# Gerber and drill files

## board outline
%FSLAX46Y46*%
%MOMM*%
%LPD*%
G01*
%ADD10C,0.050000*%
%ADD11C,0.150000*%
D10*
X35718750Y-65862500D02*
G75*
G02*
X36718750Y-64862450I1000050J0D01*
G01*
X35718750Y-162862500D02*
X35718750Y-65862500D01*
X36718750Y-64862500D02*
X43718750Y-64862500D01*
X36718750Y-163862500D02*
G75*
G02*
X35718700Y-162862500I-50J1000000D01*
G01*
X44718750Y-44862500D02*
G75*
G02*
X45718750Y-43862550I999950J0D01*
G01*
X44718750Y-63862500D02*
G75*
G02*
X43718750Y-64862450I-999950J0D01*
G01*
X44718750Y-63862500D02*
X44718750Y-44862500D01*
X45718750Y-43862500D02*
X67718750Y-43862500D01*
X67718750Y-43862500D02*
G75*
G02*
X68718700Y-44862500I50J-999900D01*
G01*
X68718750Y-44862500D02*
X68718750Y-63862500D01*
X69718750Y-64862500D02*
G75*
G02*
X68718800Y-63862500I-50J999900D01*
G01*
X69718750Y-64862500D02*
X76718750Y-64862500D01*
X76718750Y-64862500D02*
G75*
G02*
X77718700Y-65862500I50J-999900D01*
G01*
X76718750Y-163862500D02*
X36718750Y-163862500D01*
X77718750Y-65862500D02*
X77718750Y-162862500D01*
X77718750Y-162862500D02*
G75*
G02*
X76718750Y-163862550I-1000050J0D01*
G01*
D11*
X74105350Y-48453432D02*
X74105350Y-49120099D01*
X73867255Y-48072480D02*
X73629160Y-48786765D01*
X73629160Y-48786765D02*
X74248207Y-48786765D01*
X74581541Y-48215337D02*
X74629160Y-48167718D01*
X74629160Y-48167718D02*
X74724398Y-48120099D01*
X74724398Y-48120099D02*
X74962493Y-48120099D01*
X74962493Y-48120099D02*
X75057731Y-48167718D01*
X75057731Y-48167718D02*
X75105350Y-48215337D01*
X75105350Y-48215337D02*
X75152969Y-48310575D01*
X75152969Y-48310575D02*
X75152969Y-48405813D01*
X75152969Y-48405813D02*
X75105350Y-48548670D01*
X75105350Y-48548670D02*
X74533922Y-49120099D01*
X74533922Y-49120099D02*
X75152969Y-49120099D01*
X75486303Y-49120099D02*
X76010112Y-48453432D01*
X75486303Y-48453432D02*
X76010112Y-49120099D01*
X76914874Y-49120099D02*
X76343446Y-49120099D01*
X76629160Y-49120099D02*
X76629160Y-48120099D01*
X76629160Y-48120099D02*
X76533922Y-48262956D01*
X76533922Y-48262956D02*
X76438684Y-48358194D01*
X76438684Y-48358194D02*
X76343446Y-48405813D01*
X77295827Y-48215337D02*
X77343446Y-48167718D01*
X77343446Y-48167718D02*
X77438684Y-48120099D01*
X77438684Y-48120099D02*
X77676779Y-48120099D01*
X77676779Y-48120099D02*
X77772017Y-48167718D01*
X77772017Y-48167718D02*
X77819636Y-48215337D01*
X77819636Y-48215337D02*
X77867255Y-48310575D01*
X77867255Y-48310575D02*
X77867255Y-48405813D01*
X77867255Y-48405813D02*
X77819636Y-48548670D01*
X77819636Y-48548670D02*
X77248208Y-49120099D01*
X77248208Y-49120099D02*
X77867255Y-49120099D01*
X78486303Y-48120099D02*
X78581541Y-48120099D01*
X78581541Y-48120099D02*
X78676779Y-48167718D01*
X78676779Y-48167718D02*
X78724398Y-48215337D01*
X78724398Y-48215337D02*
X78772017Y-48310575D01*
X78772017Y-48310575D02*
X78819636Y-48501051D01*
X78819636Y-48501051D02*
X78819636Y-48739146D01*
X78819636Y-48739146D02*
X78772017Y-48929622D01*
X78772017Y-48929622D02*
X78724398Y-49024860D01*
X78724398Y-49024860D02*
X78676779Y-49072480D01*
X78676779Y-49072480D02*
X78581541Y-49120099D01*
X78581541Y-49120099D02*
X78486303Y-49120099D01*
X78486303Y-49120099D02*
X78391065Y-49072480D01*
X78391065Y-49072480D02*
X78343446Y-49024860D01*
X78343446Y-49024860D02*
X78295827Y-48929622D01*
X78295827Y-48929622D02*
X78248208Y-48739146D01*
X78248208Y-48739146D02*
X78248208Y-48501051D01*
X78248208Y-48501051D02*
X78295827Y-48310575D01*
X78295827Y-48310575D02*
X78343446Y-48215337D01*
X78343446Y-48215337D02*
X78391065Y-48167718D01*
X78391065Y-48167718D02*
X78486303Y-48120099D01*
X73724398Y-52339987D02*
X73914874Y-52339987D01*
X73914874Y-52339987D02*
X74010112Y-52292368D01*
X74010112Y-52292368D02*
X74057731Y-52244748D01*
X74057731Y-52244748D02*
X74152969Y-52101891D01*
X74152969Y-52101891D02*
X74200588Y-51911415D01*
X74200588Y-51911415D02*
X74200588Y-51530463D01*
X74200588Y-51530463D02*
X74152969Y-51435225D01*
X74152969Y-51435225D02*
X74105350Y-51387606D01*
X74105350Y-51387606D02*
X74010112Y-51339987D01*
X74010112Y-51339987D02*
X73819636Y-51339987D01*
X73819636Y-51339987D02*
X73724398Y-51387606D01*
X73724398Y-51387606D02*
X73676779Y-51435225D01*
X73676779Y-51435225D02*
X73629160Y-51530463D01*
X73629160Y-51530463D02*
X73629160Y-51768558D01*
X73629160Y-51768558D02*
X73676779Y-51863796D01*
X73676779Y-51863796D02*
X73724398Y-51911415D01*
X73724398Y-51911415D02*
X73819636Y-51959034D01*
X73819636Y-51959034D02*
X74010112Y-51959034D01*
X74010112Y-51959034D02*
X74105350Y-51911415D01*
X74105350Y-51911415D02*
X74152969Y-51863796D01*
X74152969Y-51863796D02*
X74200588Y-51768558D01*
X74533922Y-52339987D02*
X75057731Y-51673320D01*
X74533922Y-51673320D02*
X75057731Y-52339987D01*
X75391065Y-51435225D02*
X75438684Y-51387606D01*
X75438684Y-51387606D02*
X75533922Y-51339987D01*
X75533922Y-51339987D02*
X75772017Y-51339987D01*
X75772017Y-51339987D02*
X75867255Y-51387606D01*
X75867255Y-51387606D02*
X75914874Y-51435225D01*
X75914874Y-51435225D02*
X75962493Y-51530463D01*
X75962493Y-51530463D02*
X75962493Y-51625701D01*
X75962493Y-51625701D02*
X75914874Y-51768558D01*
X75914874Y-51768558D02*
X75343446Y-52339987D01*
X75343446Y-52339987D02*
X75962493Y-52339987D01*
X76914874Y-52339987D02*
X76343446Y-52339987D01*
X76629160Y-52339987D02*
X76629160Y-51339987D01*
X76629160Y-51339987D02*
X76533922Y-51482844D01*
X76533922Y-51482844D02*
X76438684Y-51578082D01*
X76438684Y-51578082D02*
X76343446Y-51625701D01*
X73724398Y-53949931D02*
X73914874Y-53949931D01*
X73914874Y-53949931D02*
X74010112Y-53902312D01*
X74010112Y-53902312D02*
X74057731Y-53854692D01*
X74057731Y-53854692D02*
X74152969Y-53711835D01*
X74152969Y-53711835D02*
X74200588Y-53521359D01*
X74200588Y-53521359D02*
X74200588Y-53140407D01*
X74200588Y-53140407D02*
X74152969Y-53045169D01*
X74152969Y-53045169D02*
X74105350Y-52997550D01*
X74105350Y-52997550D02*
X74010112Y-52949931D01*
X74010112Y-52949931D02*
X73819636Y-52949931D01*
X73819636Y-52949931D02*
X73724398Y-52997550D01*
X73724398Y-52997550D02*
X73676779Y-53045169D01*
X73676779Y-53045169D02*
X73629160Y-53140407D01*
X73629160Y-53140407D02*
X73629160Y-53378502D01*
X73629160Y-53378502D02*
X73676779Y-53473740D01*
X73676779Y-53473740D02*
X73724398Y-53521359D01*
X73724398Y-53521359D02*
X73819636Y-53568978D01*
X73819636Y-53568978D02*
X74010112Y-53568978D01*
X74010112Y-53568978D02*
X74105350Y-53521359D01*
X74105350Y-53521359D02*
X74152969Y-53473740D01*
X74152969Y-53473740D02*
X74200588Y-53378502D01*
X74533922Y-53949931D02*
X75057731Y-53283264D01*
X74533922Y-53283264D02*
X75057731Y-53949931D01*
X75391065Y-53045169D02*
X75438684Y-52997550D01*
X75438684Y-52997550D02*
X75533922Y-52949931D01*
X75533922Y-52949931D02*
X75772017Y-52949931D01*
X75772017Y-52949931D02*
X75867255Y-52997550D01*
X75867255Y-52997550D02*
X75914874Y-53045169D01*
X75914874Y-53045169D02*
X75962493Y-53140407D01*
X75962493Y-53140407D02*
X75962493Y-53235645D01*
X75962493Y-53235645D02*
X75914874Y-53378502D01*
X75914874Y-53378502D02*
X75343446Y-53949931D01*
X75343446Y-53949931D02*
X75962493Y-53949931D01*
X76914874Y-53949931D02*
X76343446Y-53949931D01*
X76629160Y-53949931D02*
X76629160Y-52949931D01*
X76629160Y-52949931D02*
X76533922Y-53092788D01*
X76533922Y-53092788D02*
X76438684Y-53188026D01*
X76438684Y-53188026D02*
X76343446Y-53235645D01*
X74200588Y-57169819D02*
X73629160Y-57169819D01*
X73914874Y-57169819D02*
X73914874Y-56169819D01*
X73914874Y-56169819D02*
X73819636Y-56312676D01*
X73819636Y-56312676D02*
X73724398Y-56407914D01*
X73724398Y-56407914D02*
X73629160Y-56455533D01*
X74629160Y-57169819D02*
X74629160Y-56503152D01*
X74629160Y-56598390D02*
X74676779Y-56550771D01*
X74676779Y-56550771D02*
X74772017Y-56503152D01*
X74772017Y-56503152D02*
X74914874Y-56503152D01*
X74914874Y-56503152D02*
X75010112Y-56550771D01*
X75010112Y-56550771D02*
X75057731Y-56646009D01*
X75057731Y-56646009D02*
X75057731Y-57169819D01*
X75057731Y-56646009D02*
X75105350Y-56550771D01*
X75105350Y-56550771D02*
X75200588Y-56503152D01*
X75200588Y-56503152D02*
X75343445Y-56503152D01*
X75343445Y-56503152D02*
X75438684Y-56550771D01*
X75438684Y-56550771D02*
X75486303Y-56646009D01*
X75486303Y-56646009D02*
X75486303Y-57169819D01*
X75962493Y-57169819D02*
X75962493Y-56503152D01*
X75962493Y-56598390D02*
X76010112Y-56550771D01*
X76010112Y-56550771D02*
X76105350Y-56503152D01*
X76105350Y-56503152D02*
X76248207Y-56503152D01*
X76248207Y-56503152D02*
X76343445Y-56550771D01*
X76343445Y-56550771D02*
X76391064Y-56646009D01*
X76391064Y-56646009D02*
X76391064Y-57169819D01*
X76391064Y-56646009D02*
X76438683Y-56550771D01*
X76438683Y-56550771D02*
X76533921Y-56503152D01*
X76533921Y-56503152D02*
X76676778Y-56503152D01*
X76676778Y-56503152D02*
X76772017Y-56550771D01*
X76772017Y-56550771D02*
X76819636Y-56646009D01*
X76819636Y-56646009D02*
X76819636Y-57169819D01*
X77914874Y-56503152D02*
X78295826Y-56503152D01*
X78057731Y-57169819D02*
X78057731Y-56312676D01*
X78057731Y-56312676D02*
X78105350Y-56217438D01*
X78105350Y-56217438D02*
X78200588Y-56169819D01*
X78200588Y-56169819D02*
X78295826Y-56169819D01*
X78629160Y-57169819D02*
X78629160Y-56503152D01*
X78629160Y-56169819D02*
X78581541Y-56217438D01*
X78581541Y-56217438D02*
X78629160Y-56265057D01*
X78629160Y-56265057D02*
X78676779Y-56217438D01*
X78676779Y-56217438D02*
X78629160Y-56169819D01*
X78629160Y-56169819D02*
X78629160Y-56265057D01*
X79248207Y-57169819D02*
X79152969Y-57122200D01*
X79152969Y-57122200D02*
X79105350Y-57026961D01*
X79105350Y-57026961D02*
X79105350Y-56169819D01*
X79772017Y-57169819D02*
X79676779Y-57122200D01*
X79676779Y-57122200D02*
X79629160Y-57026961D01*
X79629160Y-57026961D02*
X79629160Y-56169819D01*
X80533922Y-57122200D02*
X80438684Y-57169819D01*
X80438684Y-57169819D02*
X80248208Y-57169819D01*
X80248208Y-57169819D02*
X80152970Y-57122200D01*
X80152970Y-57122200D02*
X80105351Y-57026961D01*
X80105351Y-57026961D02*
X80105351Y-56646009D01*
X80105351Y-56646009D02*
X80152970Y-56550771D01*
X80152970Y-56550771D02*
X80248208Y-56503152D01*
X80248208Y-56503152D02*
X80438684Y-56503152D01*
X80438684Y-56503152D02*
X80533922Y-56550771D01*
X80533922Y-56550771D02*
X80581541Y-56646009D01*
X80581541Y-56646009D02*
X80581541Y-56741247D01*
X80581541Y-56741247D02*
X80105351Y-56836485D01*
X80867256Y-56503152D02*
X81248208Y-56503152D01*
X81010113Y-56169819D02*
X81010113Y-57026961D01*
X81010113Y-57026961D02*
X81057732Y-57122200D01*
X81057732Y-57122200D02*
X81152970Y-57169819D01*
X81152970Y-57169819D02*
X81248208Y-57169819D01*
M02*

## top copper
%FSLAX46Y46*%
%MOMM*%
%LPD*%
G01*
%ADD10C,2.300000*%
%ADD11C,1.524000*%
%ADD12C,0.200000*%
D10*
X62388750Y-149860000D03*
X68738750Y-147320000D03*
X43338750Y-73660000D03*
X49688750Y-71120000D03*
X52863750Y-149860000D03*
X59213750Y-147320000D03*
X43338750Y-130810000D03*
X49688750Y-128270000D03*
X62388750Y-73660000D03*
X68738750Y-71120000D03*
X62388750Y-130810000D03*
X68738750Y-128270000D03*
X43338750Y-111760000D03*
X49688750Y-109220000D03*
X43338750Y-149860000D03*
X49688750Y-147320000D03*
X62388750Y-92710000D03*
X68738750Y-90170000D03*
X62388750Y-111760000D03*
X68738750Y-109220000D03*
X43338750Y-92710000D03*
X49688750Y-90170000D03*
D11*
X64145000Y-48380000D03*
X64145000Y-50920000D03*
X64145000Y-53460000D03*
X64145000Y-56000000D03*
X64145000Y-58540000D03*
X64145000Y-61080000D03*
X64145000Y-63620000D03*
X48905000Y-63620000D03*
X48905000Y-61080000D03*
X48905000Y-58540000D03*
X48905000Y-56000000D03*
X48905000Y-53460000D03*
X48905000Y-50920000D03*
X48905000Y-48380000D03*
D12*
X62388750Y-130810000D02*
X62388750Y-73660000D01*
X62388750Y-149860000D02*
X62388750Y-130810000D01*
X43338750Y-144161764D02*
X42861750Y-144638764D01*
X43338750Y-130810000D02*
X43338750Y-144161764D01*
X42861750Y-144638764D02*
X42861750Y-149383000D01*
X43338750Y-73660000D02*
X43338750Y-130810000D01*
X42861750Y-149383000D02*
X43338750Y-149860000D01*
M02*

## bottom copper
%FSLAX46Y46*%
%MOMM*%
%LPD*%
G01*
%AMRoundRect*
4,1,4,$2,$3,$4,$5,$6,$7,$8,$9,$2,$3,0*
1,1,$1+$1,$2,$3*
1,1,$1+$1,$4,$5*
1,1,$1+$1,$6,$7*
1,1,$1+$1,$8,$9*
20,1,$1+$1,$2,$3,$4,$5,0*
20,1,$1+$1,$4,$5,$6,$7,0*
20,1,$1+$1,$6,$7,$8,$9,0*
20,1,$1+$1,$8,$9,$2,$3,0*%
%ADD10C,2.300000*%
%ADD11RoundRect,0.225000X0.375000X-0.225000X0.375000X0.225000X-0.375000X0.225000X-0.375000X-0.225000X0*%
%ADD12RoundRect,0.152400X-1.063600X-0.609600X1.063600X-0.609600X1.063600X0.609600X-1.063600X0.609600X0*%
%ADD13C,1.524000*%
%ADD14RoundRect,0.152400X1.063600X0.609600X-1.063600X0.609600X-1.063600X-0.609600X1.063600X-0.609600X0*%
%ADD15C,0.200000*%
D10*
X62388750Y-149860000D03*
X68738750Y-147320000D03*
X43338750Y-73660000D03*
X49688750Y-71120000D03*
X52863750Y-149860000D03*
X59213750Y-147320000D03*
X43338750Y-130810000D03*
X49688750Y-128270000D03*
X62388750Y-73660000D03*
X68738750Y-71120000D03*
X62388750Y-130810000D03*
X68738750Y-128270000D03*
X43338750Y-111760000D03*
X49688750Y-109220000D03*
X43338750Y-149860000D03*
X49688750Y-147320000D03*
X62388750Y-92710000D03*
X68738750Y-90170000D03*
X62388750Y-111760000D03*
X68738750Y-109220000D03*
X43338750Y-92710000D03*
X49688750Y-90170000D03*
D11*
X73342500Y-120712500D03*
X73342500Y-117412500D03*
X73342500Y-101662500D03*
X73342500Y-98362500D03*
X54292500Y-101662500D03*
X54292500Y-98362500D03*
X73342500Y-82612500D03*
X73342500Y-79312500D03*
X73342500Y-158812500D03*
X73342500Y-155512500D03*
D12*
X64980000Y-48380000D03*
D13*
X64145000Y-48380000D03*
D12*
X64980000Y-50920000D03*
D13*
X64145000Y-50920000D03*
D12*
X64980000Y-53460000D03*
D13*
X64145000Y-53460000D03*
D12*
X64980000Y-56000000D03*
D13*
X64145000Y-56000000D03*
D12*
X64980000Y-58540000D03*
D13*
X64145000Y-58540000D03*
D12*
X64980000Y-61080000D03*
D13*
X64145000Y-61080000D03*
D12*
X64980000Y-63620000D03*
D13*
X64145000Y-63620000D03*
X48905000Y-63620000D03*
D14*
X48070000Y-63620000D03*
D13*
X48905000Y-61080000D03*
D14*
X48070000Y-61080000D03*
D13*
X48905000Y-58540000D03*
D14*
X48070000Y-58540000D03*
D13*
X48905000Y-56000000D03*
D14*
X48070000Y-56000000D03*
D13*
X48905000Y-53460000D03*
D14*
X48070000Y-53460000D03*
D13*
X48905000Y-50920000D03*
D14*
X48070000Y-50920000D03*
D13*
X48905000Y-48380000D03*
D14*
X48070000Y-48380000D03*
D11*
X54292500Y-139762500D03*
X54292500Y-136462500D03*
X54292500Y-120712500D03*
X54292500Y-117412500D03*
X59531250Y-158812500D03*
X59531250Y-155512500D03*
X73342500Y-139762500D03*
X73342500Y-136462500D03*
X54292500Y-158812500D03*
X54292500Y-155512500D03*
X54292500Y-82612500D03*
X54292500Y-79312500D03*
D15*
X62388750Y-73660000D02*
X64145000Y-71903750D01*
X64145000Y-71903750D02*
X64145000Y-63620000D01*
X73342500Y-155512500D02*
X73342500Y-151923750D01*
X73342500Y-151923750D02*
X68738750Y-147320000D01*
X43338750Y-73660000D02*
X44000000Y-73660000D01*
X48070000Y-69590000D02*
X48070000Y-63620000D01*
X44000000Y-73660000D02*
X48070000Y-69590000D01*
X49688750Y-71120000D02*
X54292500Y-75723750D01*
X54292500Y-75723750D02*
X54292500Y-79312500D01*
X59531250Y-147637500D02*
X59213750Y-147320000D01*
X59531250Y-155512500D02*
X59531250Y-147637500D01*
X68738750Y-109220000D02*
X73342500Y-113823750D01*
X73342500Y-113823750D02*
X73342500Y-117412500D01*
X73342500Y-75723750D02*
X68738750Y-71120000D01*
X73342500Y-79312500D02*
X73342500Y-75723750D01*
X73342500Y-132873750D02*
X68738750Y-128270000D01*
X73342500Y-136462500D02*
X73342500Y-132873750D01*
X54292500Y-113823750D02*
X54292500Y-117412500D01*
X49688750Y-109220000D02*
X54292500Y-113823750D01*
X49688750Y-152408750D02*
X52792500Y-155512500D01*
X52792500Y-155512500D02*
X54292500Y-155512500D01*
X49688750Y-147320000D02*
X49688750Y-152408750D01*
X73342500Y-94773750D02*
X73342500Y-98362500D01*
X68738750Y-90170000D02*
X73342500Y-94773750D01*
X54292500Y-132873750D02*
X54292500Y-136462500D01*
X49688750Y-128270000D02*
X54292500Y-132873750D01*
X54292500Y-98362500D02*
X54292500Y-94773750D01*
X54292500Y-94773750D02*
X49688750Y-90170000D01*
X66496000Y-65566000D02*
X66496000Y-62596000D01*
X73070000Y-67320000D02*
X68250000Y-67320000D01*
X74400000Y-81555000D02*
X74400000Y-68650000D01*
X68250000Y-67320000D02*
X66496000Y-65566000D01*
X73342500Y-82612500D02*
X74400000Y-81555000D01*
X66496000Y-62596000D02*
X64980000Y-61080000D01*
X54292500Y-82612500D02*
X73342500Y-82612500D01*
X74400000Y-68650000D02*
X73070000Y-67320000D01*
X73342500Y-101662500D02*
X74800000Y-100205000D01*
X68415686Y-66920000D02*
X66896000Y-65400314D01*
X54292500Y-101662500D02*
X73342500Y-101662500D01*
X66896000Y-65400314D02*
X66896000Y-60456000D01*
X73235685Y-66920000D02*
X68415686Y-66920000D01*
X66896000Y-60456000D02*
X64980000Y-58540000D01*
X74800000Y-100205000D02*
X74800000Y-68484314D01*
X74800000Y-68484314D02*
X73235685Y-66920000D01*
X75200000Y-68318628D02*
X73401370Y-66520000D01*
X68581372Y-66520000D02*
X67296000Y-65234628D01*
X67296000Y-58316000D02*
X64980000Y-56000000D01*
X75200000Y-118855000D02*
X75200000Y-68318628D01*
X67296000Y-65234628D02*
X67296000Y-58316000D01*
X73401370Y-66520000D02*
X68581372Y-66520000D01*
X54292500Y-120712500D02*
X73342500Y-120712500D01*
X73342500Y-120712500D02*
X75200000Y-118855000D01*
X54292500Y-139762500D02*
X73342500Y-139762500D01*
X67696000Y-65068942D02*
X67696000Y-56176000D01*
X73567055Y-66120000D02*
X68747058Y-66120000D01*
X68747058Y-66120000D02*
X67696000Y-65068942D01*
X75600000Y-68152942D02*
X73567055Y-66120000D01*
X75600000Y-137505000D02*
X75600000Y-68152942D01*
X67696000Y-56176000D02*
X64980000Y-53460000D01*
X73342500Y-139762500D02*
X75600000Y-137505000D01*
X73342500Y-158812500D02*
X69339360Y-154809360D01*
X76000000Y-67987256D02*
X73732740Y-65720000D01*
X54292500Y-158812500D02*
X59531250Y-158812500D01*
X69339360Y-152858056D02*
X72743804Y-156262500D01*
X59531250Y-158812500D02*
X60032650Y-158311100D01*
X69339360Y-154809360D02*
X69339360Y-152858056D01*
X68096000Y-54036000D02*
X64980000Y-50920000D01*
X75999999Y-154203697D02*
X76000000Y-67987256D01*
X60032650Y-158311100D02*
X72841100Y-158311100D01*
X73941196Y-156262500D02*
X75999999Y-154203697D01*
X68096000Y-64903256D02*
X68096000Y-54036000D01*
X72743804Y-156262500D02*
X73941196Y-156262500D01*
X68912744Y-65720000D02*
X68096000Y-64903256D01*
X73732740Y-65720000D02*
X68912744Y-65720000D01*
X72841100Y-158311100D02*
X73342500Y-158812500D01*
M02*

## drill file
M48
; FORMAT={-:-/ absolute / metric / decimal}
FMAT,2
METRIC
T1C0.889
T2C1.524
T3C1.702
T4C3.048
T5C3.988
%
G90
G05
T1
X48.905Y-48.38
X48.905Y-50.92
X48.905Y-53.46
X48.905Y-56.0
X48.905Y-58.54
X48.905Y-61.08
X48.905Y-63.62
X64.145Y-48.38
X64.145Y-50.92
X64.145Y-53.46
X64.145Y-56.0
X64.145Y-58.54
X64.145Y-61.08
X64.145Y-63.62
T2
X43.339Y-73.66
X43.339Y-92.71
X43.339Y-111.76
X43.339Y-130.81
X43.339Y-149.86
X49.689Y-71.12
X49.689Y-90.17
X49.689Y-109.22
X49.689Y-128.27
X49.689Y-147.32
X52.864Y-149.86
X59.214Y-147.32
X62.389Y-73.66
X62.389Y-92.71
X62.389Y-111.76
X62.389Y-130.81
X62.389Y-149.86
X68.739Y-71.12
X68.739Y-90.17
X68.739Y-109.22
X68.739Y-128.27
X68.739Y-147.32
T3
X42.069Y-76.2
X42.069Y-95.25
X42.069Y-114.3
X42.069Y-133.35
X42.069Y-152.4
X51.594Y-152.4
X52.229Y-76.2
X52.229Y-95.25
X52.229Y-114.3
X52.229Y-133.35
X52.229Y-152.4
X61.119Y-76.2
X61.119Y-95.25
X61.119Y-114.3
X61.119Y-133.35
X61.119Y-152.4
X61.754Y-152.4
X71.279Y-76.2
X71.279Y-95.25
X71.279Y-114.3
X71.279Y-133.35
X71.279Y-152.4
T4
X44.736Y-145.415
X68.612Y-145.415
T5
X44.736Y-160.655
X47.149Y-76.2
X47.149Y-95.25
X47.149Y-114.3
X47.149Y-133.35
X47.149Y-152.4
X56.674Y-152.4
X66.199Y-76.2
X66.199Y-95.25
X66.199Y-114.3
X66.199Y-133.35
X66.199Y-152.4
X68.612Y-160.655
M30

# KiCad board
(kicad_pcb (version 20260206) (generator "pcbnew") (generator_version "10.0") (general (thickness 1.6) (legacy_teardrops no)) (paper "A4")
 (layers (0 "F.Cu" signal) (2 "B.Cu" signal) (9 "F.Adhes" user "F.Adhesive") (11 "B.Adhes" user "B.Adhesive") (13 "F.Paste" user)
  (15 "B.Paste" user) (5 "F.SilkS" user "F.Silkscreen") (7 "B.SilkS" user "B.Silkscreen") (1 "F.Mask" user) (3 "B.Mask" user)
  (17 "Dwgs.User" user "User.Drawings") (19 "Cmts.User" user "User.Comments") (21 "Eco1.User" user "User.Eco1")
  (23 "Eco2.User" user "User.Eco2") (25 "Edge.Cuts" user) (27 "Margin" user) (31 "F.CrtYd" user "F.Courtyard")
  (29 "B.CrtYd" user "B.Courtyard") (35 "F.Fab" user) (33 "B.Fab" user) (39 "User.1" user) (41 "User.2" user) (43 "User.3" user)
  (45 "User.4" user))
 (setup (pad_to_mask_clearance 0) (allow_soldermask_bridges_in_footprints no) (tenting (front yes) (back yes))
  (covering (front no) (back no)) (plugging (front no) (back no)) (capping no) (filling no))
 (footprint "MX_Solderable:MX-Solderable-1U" (layer "F.Cu") (at 66.19875 152.4)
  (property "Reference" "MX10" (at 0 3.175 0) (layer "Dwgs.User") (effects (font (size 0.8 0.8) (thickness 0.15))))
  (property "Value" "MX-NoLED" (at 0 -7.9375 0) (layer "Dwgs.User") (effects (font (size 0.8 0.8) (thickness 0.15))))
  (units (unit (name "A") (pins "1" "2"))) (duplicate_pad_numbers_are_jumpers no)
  (pad "" np_thru_hole circle (at -5.08 0 48.099) (size 1.7018 1.7018) (drill 1.7018) (layers "*.Cu" "*.Mask"))
  (pad "" np_thru_hole circle (at 0 0) (size 3.9878 3.9878) (drill 3.9878) (layers "*.Cu" "*.Mask"))
  (pad "" np_thru_hole circle (at 5.08 0 48.099) (size 1.7018 1.7018) (drill 1.7018) (layers "*.Cu" "*.Mask"))
  (pad "1" thru_hole circle (at -3.81 -2.54) (size 2.3 2.3) (drill 1.524) (layers "*.Cu" "B.Mask") (remove_unused_layers no) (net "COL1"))
  (pad "2" thru_hole circle (at 2.54 -5.08) (size 2.3 2.3) (drill 1.524) (layers "*.Cu" "B.Mask") (remove_unused_layers no)
   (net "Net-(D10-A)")))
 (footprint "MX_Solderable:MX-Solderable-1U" (layer "F.Cu") (at 47.14875 76.2)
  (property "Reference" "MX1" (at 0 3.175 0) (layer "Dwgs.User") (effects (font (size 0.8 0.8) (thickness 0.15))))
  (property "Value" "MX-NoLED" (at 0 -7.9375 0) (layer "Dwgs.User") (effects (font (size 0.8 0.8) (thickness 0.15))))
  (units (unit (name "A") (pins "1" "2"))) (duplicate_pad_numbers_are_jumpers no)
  (pad "" np_thru_hole circle (at -5.08 0 48.099) (size 1.7018 1.7018) (drill 1.7018) (layers "*.Cu" "*.Mask"))
  (pad "" np_thru_hole circle (at 0 0) (size 3.9878 3.9878) (drill 3.9878) (layers "*.Cu" "*.Mask"))
  (pad "" np_thru_hole circle (at 5.08 0 48.099) (size 1.7018 1.7018) (drill 1.7018) (layers "*.Cu" "*.Mask"))
  (pad "1" thru_hole circle (at -3.81 -2.54) (size 2.3 2.3) (drill 1.524) (layers "*.Cu" "B.Mask") (remove_unused_layers no) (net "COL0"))
  (pad "2" thru_hole circle (at 2.54 -5.08) (size 2.3 2.3) (drill 1.524) (layers "*.Cu" "B.Mask") (remove_unused_layers no)
   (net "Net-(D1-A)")))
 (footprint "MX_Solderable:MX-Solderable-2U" (layer "F.Cu") (at 56.67375 152.4)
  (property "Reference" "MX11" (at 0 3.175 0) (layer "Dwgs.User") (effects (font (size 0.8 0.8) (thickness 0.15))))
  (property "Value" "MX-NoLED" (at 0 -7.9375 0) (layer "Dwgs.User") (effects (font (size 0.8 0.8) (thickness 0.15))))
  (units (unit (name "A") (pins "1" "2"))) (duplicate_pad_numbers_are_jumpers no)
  (pad "" np_thru_hole circle (at -11.938 -6.985) (size 3.048 3.048) (drill 3.048) (layers "*.Cu" "*.Mask"))
  (pad "" np_thru_hole circle (at -11.938 8.255) (size 3.9878 3.9878) (drill 3.9878) (layers "*.Cu" "*.Mask"))
  (pad "" np_thru_hole circle (at -5.08 0 48.099) (size 1.7018 1.7018) (drill 1.7018) (layers "*.Cu" "*.Mask"))
  (pad "" np_thru_hole circle (at 0 0) (size 3.9878 3.9878) (drill 3.9878) (layers "*.Cu" "*.Mask"))
  (pad "" np_thru_hole circle (at 5.08 0 48.099) (size 1.7018 1.7018) (drill 1.7018) (layers "*.Cu" "*.Mask"))
  (pad "" np_thru_hole circle (at 11.938 -6.985) (size 3.048 3.048) (drill 3.048) (layers "*.Cu" "*.Mask"))
  (pad "" np_thru_hole circle (at 11.938 8.255) (size 3.9878 3.9878) (drill 3.9878) (layers "*.Cu" "*.Mask"))
  (pad "1" thru_hole circle (at -3.81 -2.54) (size 2.3 2.3) (drill 1.524) (layers "*.Cu" "B.Mask") (remove_unused_layers no)
   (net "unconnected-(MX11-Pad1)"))
  (pad "2" thru_hole circle (at 2.54 -5.08) (size 2.3 2.3) (drill 1.524) (layers "*.Cu" "B.Mask") (remove_unused_layers no)
   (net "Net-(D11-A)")))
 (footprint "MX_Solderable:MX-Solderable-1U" (layer "F.Cu") (at 47.14875 133.35)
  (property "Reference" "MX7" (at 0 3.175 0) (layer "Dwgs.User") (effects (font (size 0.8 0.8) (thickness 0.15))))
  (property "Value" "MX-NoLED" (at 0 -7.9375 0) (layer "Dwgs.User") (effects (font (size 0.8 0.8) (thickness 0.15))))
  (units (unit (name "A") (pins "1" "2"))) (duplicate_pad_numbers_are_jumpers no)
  (pad "" np_thru_hole circle (at -5.08 0 48.099) (size 1.7018 1.7018) (drill 1.7018) (layers "*.Cu" "*.Mask"))
  (pad "" np_thru_hole circle (at 0 0) (size 3.9878 3.9878) (drill 3.9878) (layers "*.Cu" "*.Mask"))
  (pad "" np_thru_hole circle (at 5.08 0 48.099) (size 1.7018 1.7018) (drill 1.7018) (layers "*.Cu" "*.Mask"))
  (pad "1" thru_hole circle (at -3.81 -2.54) (size 2.3 2.3) (drill 1.524) (layers "*.Cu" "B.Mask") (remove_unused_layers no) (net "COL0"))
  (pad "2" thru_hole circle (at 2.54 -5.08) (size 2.3 2.3) (drill 1.524) (layers "*.Cu" "B.Mask") (remove_unused_layers no)
   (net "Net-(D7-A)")))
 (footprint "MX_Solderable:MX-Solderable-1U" (layer "F.Cu") (at 66.19875 76.2)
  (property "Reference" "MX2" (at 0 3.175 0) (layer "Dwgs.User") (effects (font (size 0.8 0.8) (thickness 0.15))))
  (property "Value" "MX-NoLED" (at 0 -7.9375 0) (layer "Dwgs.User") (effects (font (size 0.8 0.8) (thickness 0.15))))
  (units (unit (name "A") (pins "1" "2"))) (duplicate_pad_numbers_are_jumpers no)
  (pad "" np_thru_hole circle (at -5.08 0 48.099) (size 1.7018 1.7018) (drill 1.7018) (layers "*.Cu" "*.Mask"))
  (pad "" np_thru_hole circle (at 0 0) (size 3.9878 3.9878) (drill 3.9878) (layers "*.Cu" "*.Mask"))
  (pad "" np_thru_hole circle (at 5.08 0 48.099) (size 1.7018 1.7018) (drill 1.7018) (layers "*.Cu" "*.Mask"))
  (pad "1" thru_hole circle (at -3.81 -2.54) (size 2.3 2.3) (drill 1.524) (layers "*.Cu" "B.Mask") (remove_unused_layers no) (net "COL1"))
  (pad "2" thru_hole circle (at 2.54 -5.08) (size 2.3 2.3) (drill 1.524) (layers "*.Cu" "B.Mask") (remove_unused_layers no)
   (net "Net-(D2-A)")))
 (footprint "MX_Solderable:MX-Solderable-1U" (layer "F.Cu") (at 66.19875 133.35)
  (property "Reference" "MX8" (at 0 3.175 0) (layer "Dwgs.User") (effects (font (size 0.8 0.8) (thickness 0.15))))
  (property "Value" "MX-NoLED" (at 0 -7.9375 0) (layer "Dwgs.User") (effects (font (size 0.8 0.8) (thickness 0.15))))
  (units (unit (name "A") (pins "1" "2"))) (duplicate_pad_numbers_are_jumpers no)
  (pad "" np_thru_hole circle (at -5.08 0 48.099) (size 1.7018 1.7018) (drill 1.7018) (layers "*.Cu" "*.Mask"))
  (pad "" np_thru_hole circle (at 0 0) (size 3.9878 3.9878) (drill 3.9878) (layers "*.Cu" "*.Mask"))
  (pad "" np_thru_hole circle (at 5.08 0 48.099) (size 1.7018 1.7018) (drill 1.7018) (layers "*.Cu" "*.Mask"))
  (pad "1" thru_hole circle (at -3.81 -2.54) (size 2.3 2.3) (drill 1.524) (layers "*.Cu" "B.Mask") (remove_unused_layers no) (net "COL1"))
  (pad "2" thru_hole circle (at 2.54 -5.08) (size 2.3 2.3) (drill 1.524) (layers "*.Cu" "B.Mask") (remove_unused_layers no)
   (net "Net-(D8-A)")))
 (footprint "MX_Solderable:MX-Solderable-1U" (layer "F.Cu") (at 47.14875 114.3)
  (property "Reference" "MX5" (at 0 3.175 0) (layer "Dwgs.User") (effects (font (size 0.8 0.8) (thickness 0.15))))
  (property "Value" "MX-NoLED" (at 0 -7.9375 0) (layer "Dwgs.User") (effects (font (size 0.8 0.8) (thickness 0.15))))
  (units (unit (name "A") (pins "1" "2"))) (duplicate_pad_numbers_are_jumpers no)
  (pad "" np_thru_hole circle (at -5.08 0 48.099) (size 1.7018 1.7018) (drill 1.7018) (layers "*.Cu" "*.Mask"))
  (pad "" np_thru_hole circle (at 0 0) (size 3.9878 3.9878) (drill 3.9878) (layers "*.Cu" "*.Mask"))
  (pad "" np_thru_hole circle (at 5.08 0 48.099) (size 1.7018 1.7018) (drill 1.7018) (layers "*.Cu" "*.Mask"))
  (pad "1" thru_hole circle (at -3.81 -2.54) (size 2.3 2.3) (drill 1.524) (layers "*.Cu" "B.Mask") (remove_unused_layers no) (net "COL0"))
  (pad "2" thru_hole circle (at 2.54 -5.08) (size 2.3 2.3) (drill 1.524) (layers "*.Cu" "B.Mask") (remove_unused_layers no)
   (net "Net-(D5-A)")))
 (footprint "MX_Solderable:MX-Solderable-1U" (layer "F.Cu") (at 47.14875 152.4)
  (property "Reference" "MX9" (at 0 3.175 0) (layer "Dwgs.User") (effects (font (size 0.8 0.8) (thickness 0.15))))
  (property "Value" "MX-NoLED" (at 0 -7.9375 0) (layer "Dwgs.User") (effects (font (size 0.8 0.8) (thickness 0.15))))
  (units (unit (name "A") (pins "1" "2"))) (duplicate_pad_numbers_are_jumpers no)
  (pad "" np_thru_hole circle (at -5.08 0 48.099) (size 1.7018 1.7018) (drill 1.7018) (layers "*.Cu" "*.Mask"))
  (pad "" np_thru_hole circle (at 0 0) (size 3.9878 3.9878) (drill 3.9878) (layers "*.Cu" "*.Mask"))
  (pad "" np_thru_hole circle (at 5.08 0 48.099) (size 1.7018 1.7018) (drill 1.7018) (layers "*.Cu" "*.Mask"))
  (pad "1" thru_hole circle (at -3.81 -2.54) (size 2.3 2.3) (drill 1.524) (layers "*.Cu" "B.Mask") (remove_unused_layers no) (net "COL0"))
  (pad "2" thru_hole circle (at 2.54 -5.08) (size 2.3 2.3) (drill 1.524) (layers "*.Cu" "B.Mask") (remove_unused_layers no)
   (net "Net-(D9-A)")))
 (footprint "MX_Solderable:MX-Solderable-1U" (layer "F.Cu") (at 66.19875 95.25)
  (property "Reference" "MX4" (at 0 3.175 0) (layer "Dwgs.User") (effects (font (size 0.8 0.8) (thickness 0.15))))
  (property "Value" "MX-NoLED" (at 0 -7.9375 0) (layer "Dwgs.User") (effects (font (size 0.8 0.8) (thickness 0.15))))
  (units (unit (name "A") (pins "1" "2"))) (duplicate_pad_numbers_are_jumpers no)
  (pad "" np_thru_hole circle (at -5.08 0 48.099) (size 1.7018 1.7018) (drill 1.7018) (layers "*.Cu" "*.Mask"))
  (pad "" np_thru_hole circle (at 0 0) (size 3.9878 3.9878) (drill 3.9878) (layers "*.Cu" "*.Mask"))
  (pad "" np_thru_hole circle (at 5.08 0 48.099) (size 1.7018 1.7018) (drill 1.7018) (layers "*.Cu" "*.Mask"))
  (pad "1" thru_hole circle (at -3.81 -2.54) (size 2.3 2.3) (drill 1.524) (layers "*.Cu" "B.Mask") (remove_unused_layers no) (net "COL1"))
  (pad "2" thru_hole circle (at 2.54 -5.08) (size 2.3 2.3) (drill 1.524) (layers "*.Cu" "B.Mask") (remove_unused_layers no)
   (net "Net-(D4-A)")))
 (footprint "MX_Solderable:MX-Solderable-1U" (layer "F.Cu") (at 66.19875 114.3)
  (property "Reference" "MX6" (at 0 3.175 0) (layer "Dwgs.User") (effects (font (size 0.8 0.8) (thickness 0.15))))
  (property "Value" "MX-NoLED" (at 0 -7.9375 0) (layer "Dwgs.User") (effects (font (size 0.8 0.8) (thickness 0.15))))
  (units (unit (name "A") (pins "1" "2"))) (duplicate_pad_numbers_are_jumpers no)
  (pad "" np_thru_hole circle (at -5.08 0 48.099) (size 1.7018 1.7018) (drill 1.7018) (layers "*.Cu" "*.Mask"))
  (pad "" np_thru_hole circle (at 0 0) (size 3.9878 3.9878) (drill 3.9878) (layers "*.Cu" "*.Mask"))
  (pad "" np_thru_hole circle (at 5.08 0 48.099) (size 1.7018 1.7018) (drill 1.7018) (layers "*.Cu" "*.Mask"))
  (pad "1" thru_hole circle (at -3.81 -2.54) (size 2.3 2.3) (drill 1.524) (layers "*.Cu" "B.Mask") (remove_unused_layers no) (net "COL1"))
  (pad "2" thru_hole circle (at 2.54 -5.08) (size 2.3 2.3) (drill 1.524) (layers "*.Cu" "B.Mask") (remove_unused_layers no)
   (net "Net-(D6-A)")))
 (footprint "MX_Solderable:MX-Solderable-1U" (layer "F.Cu") (at 47.14875 95.25)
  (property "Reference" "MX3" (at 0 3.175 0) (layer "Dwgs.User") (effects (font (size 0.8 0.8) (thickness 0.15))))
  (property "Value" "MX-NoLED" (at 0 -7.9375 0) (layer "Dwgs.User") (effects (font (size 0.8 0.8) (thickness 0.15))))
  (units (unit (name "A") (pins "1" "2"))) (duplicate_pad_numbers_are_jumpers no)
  (pad "" np_thru_hole circle (at -5.08 0 48.099) (size 1.7018 1.7018) (drill 1.7018) (layers "*.Cu" "*.Mask"))
  (pad "" np_thru_hole circle (at 0 0) (size 3.9878 3.9878) (drill 3.9878) (layers "*.Cu" "*.Mask"))
  (pad "" np_thru_hole circle (at 5.08 0 48.099) (size 1.7018 1.7018) (drill 1.7018) (layers "*.Cu" "*.Mask"))
  (pad "1" thru_hole circle (at -3.81 -2.54) (size 2.3 2.3) (drill 1.524) (layers "*.Cu" "B.Mask") (remove_unused_layers no) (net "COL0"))
  (pad "2" thru_hole circle (at 2.54 -5.08) (size 2.3 2.3) (drill 1.524) (layers "*.Cu" "B.Mask") (remove_unused_layers no)
   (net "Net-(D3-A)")))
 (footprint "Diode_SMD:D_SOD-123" (layer "B.Cu") (at 73.3425 119.0625 90)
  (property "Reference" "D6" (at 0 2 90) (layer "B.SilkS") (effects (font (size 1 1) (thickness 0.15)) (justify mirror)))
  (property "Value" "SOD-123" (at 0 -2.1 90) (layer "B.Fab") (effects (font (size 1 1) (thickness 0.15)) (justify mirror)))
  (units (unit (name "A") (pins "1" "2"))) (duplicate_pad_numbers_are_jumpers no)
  (pad "1" smd roundrect (at -1.65 0 90) (size 0.9 1.2) (layers "B.Cu" "B.Mask" "B.Paste") (roundrect_rratio 0.25) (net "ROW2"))
  (pad "2" smd roundrect (at 1.65 0 90) (size 0.9 1.2) (layers "B.Cu" "B.Mask" "B.Paste") (roundrect_rratio 0.25) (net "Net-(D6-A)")))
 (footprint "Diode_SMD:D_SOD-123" (layer "B.Cu") (at 73.3425 100.0125 90)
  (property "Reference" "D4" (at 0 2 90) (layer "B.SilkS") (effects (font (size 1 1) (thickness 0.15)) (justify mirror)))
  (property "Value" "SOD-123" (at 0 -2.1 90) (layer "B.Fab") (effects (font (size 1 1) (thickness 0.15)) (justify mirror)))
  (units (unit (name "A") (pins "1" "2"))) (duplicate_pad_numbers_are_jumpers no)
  (pad "1" smd roundrect (at -1.65 0 90) (size 0.9 1.2) (layers "B.Cu" "B.Mask" "B.Paste") (roundrect_rratio 0.25) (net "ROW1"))
  (pad "2" smd roundrect (at 1.65 0 90) (size 0.9 1.2) (layers "B.Cu" "B.Mask" "B.Paste") (roundrect_rratio 0.25) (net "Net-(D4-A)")))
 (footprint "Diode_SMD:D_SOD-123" (layer "B.Cu") (at 54.2925 100.0125 90)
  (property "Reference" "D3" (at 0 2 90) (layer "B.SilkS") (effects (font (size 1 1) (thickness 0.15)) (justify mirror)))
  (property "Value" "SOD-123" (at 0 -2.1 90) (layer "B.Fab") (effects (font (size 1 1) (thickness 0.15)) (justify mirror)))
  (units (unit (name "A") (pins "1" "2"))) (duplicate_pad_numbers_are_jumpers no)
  (pad "1" smd roundrect (at -1.65 0 90) (size 0.9 1.2) (layers "B.Cu" "B.Mask" "B.Paste") (roundrect_rratio 0.25) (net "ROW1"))
  (pad "2" smd roundrect (at 1.65 0 90) (size 0.9 1.2) (layers "B.Cu" "B.Mask" "B.Paste") (roundrect_rratio 0.25) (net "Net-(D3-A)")))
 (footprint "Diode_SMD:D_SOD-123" (layer "B.Cu") (at 73.3425 80.9625 90)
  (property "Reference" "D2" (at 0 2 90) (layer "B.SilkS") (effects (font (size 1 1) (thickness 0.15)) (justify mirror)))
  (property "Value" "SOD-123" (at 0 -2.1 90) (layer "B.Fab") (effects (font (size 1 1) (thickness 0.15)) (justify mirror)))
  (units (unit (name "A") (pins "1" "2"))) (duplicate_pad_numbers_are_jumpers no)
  (pad "1" smd roundrect (at -1.65 0 90) (size 0.9 1.2) (layers "B.Cu" "B.Mask" "B.Paste") (roundrect_rratio 0.25) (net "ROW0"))
  (pad "2" smd roundrect (at 1.65 0 90) (size 0.9 1.2) (layers "B.Cu" "B.Mask" "B.Paste") (roundrect_rratio 0.25) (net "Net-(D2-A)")))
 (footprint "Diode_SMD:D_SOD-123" (layer "B.Cu") (at 73.3425 157.1625 90)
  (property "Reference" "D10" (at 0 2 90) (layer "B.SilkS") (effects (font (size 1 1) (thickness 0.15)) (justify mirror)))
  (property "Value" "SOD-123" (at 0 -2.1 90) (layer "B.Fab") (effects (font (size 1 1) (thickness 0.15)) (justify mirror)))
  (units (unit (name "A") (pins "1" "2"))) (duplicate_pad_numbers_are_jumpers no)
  (pad "1" smd roundrect (at -1.65 0 90) (size 0.9 1.2) (layers "B.Cu" "B.Mask" "B.Paste") (roundrect_rratio 0.25) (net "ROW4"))
  (pad "2" smd roundrect (at 1.65 0 90) (size 0.9 1.2) (layers "B.Cu" "B.Mask" "B.Paste") (roundrect_rratio 0.25) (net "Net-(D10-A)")))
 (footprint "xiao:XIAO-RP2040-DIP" (layer "B.Cu") (at 56.525 56 180)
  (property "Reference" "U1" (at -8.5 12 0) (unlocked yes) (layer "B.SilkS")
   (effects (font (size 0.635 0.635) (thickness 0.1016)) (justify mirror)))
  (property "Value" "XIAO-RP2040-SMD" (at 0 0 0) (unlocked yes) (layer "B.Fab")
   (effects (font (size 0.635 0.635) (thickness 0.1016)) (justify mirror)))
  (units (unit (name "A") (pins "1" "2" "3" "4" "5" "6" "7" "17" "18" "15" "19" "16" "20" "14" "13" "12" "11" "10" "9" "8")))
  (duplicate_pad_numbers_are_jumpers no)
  (pad "1" smd roundrect (at -8.455 7.62) (size 2.432 1.524) (layers "B.Cu" "B.Mask") (roundrect_rratio 0.1)
   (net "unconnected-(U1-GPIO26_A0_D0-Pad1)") (thermal_bridge_angle 45))
  (pad "1" thru_hole circle (at -7.62 7.62) (size 1.524 1.524) (drill 0.889) (layers "*.Cu" "*.Mask") (remove_unused_layers no)
   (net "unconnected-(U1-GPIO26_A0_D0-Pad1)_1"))
  (pad "2" smd roundrect (at -8.455 5.08) (size 2.432 1.524) (layers "B.Cu" "B.Mask") (roundrect_rratio 0.1) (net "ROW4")
   (thermal_bridge_angle 45))
  (pad "2" thru_hole circle (at -7.62 5.08) (size 1.524 1.524) (drill 0.889) (layers "*.Cu" "*.Mask") (remove_unused_layers no) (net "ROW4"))
  (pad "3" smd roundrect (at -8.455 2.54) (size 2.432 1.524) (layers "B.Cu" "B.Mask") (roundrect_rratio 0.1) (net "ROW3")
   (thermal_bridge_angle 45))
  (pad "3" thru_hole circle (at -7.62 2.54) (size 1.524 1.524) (drill 0.889) (layers "*.Cu" "*.Mask") (remove_unused_layers no) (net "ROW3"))
  (pad "4" smd roundrect (at -8.455 0) (size 2.432 1.524) (layers "B.Cu" "B.Mask") (roundrect_rratio 0.1) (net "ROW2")
   (thermal_bridge_angle 45))
  (pad "4" thru_hole circle (at -7.62 0) (size 1.524 1.524) (drill 0.889) (layers "*.Cu" "*.Mask") (remove_unused_layers no) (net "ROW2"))
  (pad "5" smd roundrect (at -8.455 -2.54) (size 2.432 1.524) (layers "B.Cu" "B.Mask") (roundrect_rratio 0.1) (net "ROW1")
   (thermal_bridge_angle 45))
  (pad "5" thru_hole circle (at -7.62 -2.54) (size 1.524 1.524) (drill 0.889) (layers "*.Cu" "*.Mask") (remove_unused_layers no)
   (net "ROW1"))
  (pad "6" smd roundrect (at -8.455 -5.08) (size 2.432 1.524) (layers "B.Cu" "B.Mask") (roundrect_rratio 0.1) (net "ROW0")
   (thermal_bridge_angle 45))
  (pad "6" thru_hole circle (at -7.62 -5.08) (size 1.524 1.524) (drill 0.889) (layers "*.Cu" "*.Mask") (remove_unused_layers no)
   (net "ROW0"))
  (pad "7" smd roundrect (at -8.455 -7.62) (size 2.432 1.524) (layers "B.Cu" "B.Mask") (roundrect_rratio 0.1) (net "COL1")
   (thermal_bridge_angle 45))
  (pad "7" thru_hole circle (at -7.62 -7.62) (size 1.524 1.524) (drill 0.889) (layers "*.Cu" "*.Mask") (remove_unused_layers no)
   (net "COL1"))
  (pad "8" thru_hole circle (at 7.62 -7.62 180) (size 1.524 1.524) (drill 0.889) (layers "*.Cu" "*.Mask") (remove_unused_layers no)
   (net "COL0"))
  (pad "8" smd roundrect (at 8.455 -7.62 180) (size 2.432 1.524) (layers "B.Cu" "B.Mask") (roundrect_rratio 0.1) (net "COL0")
   (thermal_bridge_angle 45))
  (pad "9" thru_hole circle (at 7.62 -5.08 180) (size 1.524 1.524) (drill 0.889) (layers "*.Cu" "*.Mask") (remove_unused_layers no)
   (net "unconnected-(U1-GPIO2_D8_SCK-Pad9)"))
  (pad "9" smd roundrect (at 8.455 -5.08 180) (size 2.432 1.524) (layers "B.Cu" "B.Mask") (roundrect_rratio 0.1)
   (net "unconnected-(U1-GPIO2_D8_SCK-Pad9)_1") (thermal_bridge_angle 45))
  (pad "10" thru_hole circle (at 7.62 -2.54 180) (size 1.524 1.524) (drill 0.889) (layers "*.Cu" "*.Mask") (remove_unused_layers no)
   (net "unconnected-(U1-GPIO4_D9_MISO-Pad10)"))
  (pad "10" smd roundrect (at 8.455 -2.54 180) (size 2.432 1.524) (layers "B.Cu" "B.Mask") (roundrect_rratio 0.1)
   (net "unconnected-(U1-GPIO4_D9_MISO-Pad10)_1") (thermal_bridge_angle 45))
  (pad "11" thru_hole circle (at 7.62 0 180) (size 1.524 1.524) (drill 0.889) (layers "*.Cu" "*.Mask") (remove_unused_layers no)
   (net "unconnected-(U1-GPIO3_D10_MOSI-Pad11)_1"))
  (pad "11" smd roundrect (at 8.455 0 180) (size 2.432 1.524) (layers "B.Cu" "B.Mask") (roundrect_rratio 0.1)
   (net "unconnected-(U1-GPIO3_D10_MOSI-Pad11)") (thermal_bridge_angle 45))
  (pad "12" thru_hole circle (at 7.62 2.54 180) (size 1.524 1.524) (drill 0.889) (layers "*.Cu" "*.Mask") (remove_unused_layers no)
   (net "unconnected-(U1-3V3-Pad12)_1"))
  (pad "12" smd roundrect (at 8.455 2.54 180) (size 2.432 1.524) (layers "B.Cu" "B.Mask") (roundrect_rratio 0.1)
   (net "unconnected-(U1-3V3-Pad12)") (thermal_bridge_angle 45))
  (pad "13" thru_hole circle (at 7.62 5.08 180) (size 1.524 1.524) (drill 0.889) (layers "*.Cu" "*.Mask") (remove_unused_layers no)
   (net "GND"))
  (pad "13" smd roundrect (at 8.455 5.08 180) (size 2.432 1.524) (layers "B.Cu" "B.Mask") (roundrect_rratio 0.1) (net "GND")
   (thermal_bridge_angle 45))
  (pad "14" thru_hole circle (at 7.62 7.62 180) (size 1.524 1.524) (drill 0.889) (layers "*.Cu" "*.Mask") (remove_unused_layers no)
   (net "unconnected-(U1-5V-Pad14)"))
  (pad "14" smd roundrect (at 8.455 7.62 180) (size 2.432 1.524) (layers "B.Cu" "B.Mask") (roundrect_rratio 0.1)
   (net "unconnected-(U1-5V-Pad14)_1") (thermal_bridge_angle 45)))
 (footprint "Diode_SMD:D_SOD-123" (layer "B.Cu") (at 54.2925 138.1125 90)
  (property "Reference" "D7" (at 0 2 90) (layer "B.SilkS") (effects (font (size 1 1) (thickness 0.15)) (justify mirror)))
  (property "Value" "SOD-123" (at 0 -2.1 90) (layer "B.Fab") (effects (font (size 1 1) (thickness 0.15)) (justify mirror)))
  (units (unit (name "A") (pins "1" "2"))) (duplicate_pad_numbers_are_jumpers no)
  (pad "1" smd roundrect (at -1.65 0 90) (size 0.9 1.2) (layers "B.Cu" "B.Mask" "B.Paste") (roundrect_rratio 0.25) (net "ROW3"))
  (pad "2" smd roundrect (at 1.65 0 90) (size 0.9 1.2) (layers "B.Cu" "B.Mask" "B.Paste") (roundrect_rratio 0.25) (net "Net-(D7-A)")))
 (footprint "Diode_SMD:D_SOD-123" (layer "B.Cu") (at 54.2925 119.0625 90)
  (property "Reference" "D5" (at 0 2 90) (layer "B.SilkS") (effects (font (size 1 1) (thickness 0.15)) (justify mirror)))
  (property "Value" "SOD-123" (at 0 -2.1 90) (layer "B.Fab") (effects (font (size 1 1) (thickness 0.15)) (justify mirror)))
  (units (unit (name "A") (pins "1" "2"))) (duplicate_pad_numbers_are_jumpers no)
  (pad "1" smd roundrect (at -1.65 0 90) (size 0.9 1.2) (layers "B.Cu" "B.Mask" "B.Paste") (roundrect_rratio 0.25) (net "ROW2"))
  (pad "2" smd roundrect (at 1.65 0 90) (size 0.9 1.2) (layers "B.Cu" "B.Mask" "B.Paste") (roundrect_rratio 0.25) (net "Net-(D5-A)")))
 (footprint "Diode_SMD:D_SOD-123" (layer "B.Cu") (at 59.53125 157.1625 90)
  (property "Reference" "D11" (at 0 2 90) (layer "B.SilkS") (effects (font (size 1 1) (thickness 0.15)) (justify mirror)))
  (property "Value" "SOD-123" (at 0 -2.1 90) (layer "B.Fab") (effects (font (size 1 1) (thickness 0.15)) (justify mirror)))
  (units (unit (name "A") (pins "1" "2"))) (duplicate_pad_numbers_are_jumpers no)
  (pad "1" smd roundrect (at -1.65 0 90) (size 0.9 1.2) (layers "B.Cu" "B.Mask" "B.Paste") (roundrect_rratio 0.25) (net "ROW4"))
  (pad "2" smd roundrect (at 1.65 0 90) (size 0.9 1.2) (layers "B.Cu" "B.Mask" "B.Paste") (roundrect_rratio 0.25) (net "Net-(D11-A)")))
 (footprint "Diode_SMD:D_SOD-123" (layer "B.Cu") (at 73.3425 138.1125 90)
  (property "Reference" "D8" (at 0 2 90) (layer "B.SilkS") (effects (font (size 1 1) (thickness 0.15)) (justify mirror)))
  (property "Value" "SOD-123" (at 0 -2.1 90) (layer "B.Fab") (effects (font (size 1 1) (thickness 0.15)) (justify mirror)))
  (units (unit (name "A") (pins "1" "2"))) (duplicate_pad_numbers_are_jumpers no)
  (pad "1" smd roundrect (at -1.65 0 90) (size 0.9 1.2) (layers "B.Cu" "B.Mask" "B.Paste") (roundrect_rratio 0.25) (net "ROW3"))
  (pad "2" smd roundrect (at 1.65 0 90) (size 0.9 1.2) (layers "B.Cu" "B.Mask" "B.Paste") (roundrect_rratio 0.25) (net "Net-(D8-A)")))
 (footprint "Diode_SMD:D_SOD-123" (layer "B.Cu") (at 54.2925 157.1625 90)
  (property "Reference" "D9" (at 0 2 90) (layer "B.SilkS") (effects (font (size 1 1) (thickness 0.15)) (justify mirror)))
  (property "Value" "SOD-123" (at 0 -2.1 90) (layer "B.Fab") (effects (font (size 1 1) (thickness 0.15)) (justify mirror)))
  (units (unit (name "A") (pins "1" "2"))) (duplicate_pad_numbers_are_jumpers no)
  (pad "1" smd roundrect (at -1.65 0 90) (size 0.9 1.2) (layers "B.Cu" "B.Mask" "B.Paste") (roundrect_rratio 0.25) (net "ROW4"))
  (pad "2" smd roundrect (at 1.65 0 90) (size 0.9 1.2) (layers "B.Cu" "B.Mask" "B.Paste") (roundrect_rratio 0.25) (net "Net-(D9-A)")))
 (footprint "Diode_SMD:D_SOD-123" (layer "B.Cu") (at 54.2925 80.9625 90)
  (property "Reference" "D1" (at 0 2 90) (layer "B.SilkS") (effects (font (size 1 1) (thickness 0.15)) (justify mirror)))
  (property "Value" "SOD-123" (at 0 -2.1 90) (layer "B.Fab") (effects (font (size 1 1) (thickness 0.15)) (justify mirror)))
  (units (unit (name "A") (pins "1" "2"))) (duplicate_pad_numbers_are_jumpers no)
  (pad "1" smd roundrect (at -1.65 0 90) (size 0.9 1.2) (layers "B.Cu" "B.Mask" "B.Paste") (roundrect_rratio 0.25) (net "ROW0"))
  (pad "2" smd roundrect (at 1.65 0 90) (size 0.9 1.2) (layers "B.Cu" "B.Mask" "B.Paste") (roundrect_rratio 0.25) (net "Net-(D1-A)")))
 (gr_arc (start 35.71875 65.8625) (mid 36.011646 65.155411) (end 36.71875 64.8625) (stroke (width 0.05) (type default)) (layer "Edge.Cuts"))
 (gr_line (start 35.71875 162.8625) (end 35.71875 65.8625) (stroke (width 0.05) (type default)) (layer "Edge.Cuts"))
 (gr_line (start 36.71875 64.8625) (end 43.71875 64.8625) (stroke (width 0.05) (type default)) (layer "Edge.Cuts"))
 (gr_arc (start 36.71875 163.8625) (mid 36.011643 163.569607) (end 35.71875 162.8625) (stroke (width 0.05) (type default))
  (layer "Edge.Cuts"))
 (gr_arc (start 44.71875 44.8625) (mid 45.011643 44.155393) (end 45.71875 43.8625) (stroke (width 0.05) (type default)) (layer "Edge.Cuts"))
 (gr_arc (start 44.71875 63.8625) (mid 44.425857 64.569607) (end 43.71875 64.8625) (stroke (width 0.05) (type default)) (layer "Edge.Cuts"))
 (gr_line (start 44.71875 63.8625) (end 44.71875 44.8625) (stroke (width 0.05) (type default)) (layer "Edge.Cuts"))
 (gr_line (start 45.71875 43.8625) (end 67.71875 43.8625) (stroke (width 0.05) (type default)) (layer "Edge.Cuts"))
 (gr_arc (start 67.71875 43.8625) (mid 68.425889 44.155376) (end 68.71875 44.8625) (stroke (width 0.05) (type default)) (layer "Edge.Cuts"))
 (gr_line (start 68.71875 44.8625) (end 68.71875 63.8625) (stroke (width 0.05) (type default)) (layer "Edge.Cuts"))
 (gr_arc (start 69.71875 64.8625) (mid 69.011611 64.569624) (end 68.71875 63.8625) (stroke (width 0.05) (type default)) (layer "Edge.Cuts"))
 (gr_line (start 69.71875 64.8625) (end 76.71875 64.8625) (stroke (width 0.05) (type default)) (layer "Edge.Cuts"))
 (gr_arc (start 76.71875 64.8625) (mid 77.425889 65.155376) (end 77.71875 65.8625) (stroke (width 0.05) (type default)) (layer "Edge.Cuts"))
 (gr_line (start 76.71875 163.8625) (end 36.71875 163.8625) (stroke (width 0.05) (type default)) (layer "Edge.Cuts"))
 (gr_line (start 77.71875 65.8625) (end 77.71875 162.8625) (stroke (width 0.05) (type default)) (layer "Edge.Cuts"))
 (gr_arc (start 77.71875 162.8625) (mid 77.425854 163.569589) (end 76.71875 163.8625) (stroke (width 0.05) (type default))
  (layer "Edge.Cuts"))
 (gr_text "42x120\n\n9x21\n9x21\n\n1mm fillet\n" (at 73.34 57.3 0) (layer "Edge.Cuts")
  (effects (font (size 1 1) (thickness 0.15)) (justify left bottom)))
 (segment (start 62.38875 130.81) (end 62.38875 73.66) (width 0.2) (layer "F.Cu") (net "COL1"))
 (segment (start 62.38875 149.86) (end 62.38875 130.81) (width 0.2) (layer "F.Cu") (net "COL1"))
 (segment (start 62.38875 73.66) (end 64.145 71.90375) (width 0.2) (layer "B.Cu") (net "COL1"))
 (segment (start 64.145 71.90375) (end 64.145 63.62) (width 0.2) (layer "B.Cu") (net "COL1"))
 (segment (start 73.3425 155.5125) (end 73.3425 151.92375) (width 0.2) (layer "B.Cu") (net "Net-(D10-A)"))
 (segment (start 73.3425 151.92375) (end 68.73875 147.32) (width 0.2) (layer "B.Cu") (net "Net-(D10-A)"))
 (segment (start 43.33875 144.161764) (end 42.86175 144.638764) (width 0.2) (layer "F.Cu") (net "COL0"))
 (segment (start 43.33875 130.81) (end 43.33875 144.161764) (width 0.2) (layer "F.Cu") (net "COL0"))
 (segment (start 42.86175 144.638764) (end 42.86175 149.383) (width 0.2) (layer "F.Cu") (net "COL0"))
 (segment (start 43.33875 73.66) (end 43.33875 130.81) (width 0.2) (layer "F.Cu") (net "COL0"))
 (segment (start 42.86175 149.383) (end 43.33875 149.86) (width 0.2) (layer "F.Cu") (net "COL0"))
 (segment (start 43.33875 73.66) (end 44 73.66) (width 0.2) (layer "B.Cu") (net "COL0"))
 (segment (start 48.07 69.59) (end 48.07 63.62) (width 0.2) (layer "B.Cu") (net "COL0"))
 (segment (start 44 73.66) (end 48.07 69.59) (width 0.2) (layer "B.Cu") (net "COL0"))
 (segment (start 49.68875 71.12) (end 54.2925 75.72375) (width 0.2) (layer "B.Cu") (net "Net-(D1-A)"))
 (segment (start 54.2925 75.72375) (end 54.2925 79.3125) (width 0.2) (layer "B.Cu") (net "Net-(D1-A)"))
 (segment (start 59.53125 147.6375) (end 59.21375 147.32) (width 0.2) (layer "B.Cu") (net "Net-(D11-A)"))
 (segment (start 59.53125 155.5125) (end 59.53125 147.6375) (width 0.2) (layer "B.Cu") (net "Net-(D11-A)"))
 (segment (start 68.73875 109.22) (end 73.3425 113.82375) (width 0.2) (layer "B.Cu") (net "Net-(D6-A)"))
 (segment (start 73.3425 113.82375) (end 73.3425 117.4125) (width 0.2) (layer "B.Cu") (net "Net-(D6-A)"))
 (segment (start 73.3425 75.72375) (end 68.73875 71.12) (width 0.2) (layer "B.Cu") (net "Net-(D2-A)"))
 (segment (start 73.3425 79.3125) (end 73.3425 75.72375) (width 0.2) (layer "B.Cu") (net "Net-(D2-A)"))
 (segment (start 73.3425 132.87375) (end 68.73875 128.27) (width 0.2) (layer "B.Cu") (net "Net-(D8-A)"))
 (segment (start 73.3425 136.4625) (end 73.3425 132.87375) (width 0.2) (layer "B.Cu") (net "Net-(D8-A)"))
 (segment (start 54.2925 113.82375) (end 54.2925 117.4125) (width 0.2) (layer "B.Cu") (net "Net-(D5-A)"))
 (segment (start 49.68875 109.22) (end 54.2925 113.82375) (width 0.2) (layer "B.Cu") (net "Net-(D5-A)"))
 (segment (start 49.68875 152.40875) (end 52.7925 155.5125) (width 0.2) (layer "B.Cu") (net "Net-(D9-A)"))
 (segment (start 52.7925 155.5125) (end 54.2925 155.5125) (width 0.2) (layer "B.Cu") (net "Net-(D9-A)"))
 (segment (start 49.68875 147.32) (end 49.68875 152.40875) (width 0.2) (layer "B.Cu") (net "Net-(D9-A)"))
 (segment (start 73.3425 94.77375) (end 73.3425 98.3625) (width 0.2) (layer "B.Cu") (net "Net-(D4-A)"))
 (segment (start 68.73875 90.17) (end 73.3425 94.77375) (width 0.2) (layer "B.Cu") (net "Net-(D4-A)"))
 (segment (start 54.2925 132.87375) (end 54.2925 136.4625) (width 0.2) (layer "B.Cu") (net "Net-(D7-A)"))
 (segment (start 49.68875 128.27) (end 54.2925 132.87375) (width 0.2) (layer "B.Cu") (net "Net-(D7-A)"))
 (segment (start 54.2925 98.3625) (end 54.2925 94.77375) (width 0.2) (layer "B.Cu") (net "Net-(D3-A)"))
 (segment (start 54.2925 94.77375) (end 49.68875 90.17) (width 0.2) (layer "B.Cu") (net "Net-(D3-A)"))
 (segment (start 66.496 65.566) (end 66.496 62.596) (width 0.2) (layer "B.Cu") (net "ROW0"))
 (segment (start 73.07 67.32) (end 68.25 67.32) (width 0.2) (layer "B.Cu") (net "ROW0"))
 (segment (start 74.4 81.555) (end 74.4 68.65) (width 0.2) (layer "B.Cu") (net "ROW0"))
 (segment (start 68.25 67.32) (end 66.496 65.566) (width 0.2) (layer "B.Cu") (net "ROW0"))
 (segment (start 73.3425 82.6125) (end 74.4 81.555) (width 0.2) (layer "B.Cu") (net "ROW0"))
 (segment (start 66.496 62.596) (end 64.98 61.08) (width 0.2) (layer "B.Cu") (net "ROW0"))
 (segment (start 54.2925 82.6125) (end 73.3425 82.6125) (width 0.2) (layer "B.Cu") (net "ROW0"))
 (segment (start 74.4 68.65) (end 73.07 67.32) (width 0.2) (layer "B.Cu") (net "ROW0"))
 (segment (start 73.3425 101.6625) (end 74.8 100.205) (width 0.2) (layer "B.Cu") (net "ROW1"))
 (segment (start 68.415686 66.92) (end 66.896 65.400314) (width 0.2) (layer "B.Cu") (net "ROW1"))
 (segment (start 54.2925 101.6625) (end 73.3425 101.6625) (width 0.2) (layer "B.Cu") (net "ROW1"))
 (segment (start 66.896 65.400314) (end 66.896 60.456) (width 0.2) (layer "B.Cu") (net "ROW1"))
 (segment (start 73.235685 66.92) (end 68.415686 66.92) (width 0.2) (layer "B.Cu") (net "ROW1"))
 (segment (start 66.896 60.456) (end 64.98 58.54) (width 0.2) (layer "B.Cu") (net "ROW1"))
 (segment (start 74.8 100.205) (end 74.8 68.484314) (width 0.2) (layer "B.Cu") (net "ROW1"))
 (segment (start 74.8 68.484314) (end 73.235685 66.92) (width 0.2) (layer "B.Cu") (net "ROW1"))
 (segment (start 75.2 68.318628) (end 73.40137 66.52) (width 0.2) (layer "B.Cu") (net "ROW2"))
 (segment (start 68.581372 66.52) (end 67.296 65.234628) (width 0.2) (layer "B.Cu") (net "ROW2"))
 (segment (start 67.296 58.316) (end 64.98 56) (width 0.2) (layer "B.Cu") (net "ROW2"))
 (segment (start 75.2 118.855) (end 75.2 68.318628) (width 0.2) (layer "B.Cu") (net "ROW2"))
 (segment (start 67.296 65.234628) (end 67.296 58.316) (width 0.2) (layer "B.Cu") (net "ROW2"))
 (segment (start 73.40137 66.52) (end 68.581372 66.52) (width 0.2) (layer "B.Cu") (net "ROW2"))
 (segment (start 54.2925 120.7125) (end 73.3425 120.7125) (width 0.2) (layer "B.Cu") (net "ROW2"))
 (segment (start 73.3425 120.7125) (end 75.2 118.855) (width 0.2) (layer "B.Cu") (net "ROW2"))
 (segment (start 54.2925 139.7625) (end 73.3425 139.7625) (width 0.2) (layer "B.Cu") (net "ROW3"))
 (segment (start 67.696 65.068942) (end 67.696 56.176) (width 0.2) (layer "B.Cu") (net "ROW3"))
 (segment (start 73.567055 66.12) (end 68.747058 66.12) (width 0.2) (layer "B.Cu") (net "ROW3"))
 (segment (start 68.747058 66.12) (end 67.696 65.068942) (width 0.2) (layer "B.Cu") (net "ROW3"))
 (segment (start 75.6 68.152942) (end 73.567055 66.12) (width 0.2) (layer "B.Cu") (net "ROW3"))
 (segment (start 75.6 137.505) (end 75.6 68.152942) (width 0.2) (layer "B.Cu") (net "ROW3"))
 (segment (start 67.696 56.176) (end 64.98 53.46) (width 0.2) (layer "B.Cu") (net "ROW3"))
 (segment (start 73.3425 139.7625) (end 75.6 137.505) (width 0.2) (layer "B.Cu") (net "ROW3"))
 (segment (start 73.3425 158.8125) (end 69.33936 154.80936) (width 0.2) (layer "B.Cu") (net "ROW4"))
 (segment (start 76 67.987256) (end 73.73274 65.72) (width 0.2) (layer "B.Cu") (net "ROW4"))
 (segment (start 54.2925 158.8125) (end 59.53125 158.8125) (width 0.2) (layer "B.Cu") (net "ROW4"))
 (segment (start 69.33936 152.858056) (end 72.743804 156.2625) (width 0.2) (layer "B.Cu") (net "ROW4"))
 (segment (start 59.53125 158.8125) (end 60.03265 158.3111) (width 0.2) (layer "B.Cu") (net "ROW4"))
 (segment (start 69.33936 154.80936) (end 69.33936 152.858056) (width 0.2) (layer "B.Cu") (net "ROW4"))
 (segment (start 68.096 54.036) (end 64.98 50.92) (width 0.2) (layer "B.Cu") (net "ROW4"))
 (segment (start 75.999999 154.203697) (end 76 67.987256) (width 0.2) (layer "B.Cu") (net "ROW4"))
 (segment (start 60.03265 158.3111) (end 72.8411 158.3111) (width 0.2) (layer "B.Cu") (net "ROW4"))
 (segment (start 73.941196 156.2625) (end 75.999999 154.203697) (width 0.2) (layer "B.Cu") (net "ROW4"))
 (segment (start 68.096 64.903256) (end 68.096 54.036) (width 0.2) (layer "B.Cu") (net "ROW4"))
 (segment (start 72.743804 156.2625) (end 73.941196 156.2625) (width 0.2) (layer "B.Cu") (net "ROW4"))
 (segment (start 68.912744 65.72) (end 68.096 64.903256) (width 0.2) (layer "B.Cu") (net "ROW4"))
 (segment (start 73.73274 65.72) (end 68.912744 65.72) (width 0.2) (layer "B.Cu") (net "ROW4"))
 (segment (start 72.8411 158.3111) (end 73.3425 158.8125) (width 0.2) (layer "B.Cu") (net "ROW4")))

